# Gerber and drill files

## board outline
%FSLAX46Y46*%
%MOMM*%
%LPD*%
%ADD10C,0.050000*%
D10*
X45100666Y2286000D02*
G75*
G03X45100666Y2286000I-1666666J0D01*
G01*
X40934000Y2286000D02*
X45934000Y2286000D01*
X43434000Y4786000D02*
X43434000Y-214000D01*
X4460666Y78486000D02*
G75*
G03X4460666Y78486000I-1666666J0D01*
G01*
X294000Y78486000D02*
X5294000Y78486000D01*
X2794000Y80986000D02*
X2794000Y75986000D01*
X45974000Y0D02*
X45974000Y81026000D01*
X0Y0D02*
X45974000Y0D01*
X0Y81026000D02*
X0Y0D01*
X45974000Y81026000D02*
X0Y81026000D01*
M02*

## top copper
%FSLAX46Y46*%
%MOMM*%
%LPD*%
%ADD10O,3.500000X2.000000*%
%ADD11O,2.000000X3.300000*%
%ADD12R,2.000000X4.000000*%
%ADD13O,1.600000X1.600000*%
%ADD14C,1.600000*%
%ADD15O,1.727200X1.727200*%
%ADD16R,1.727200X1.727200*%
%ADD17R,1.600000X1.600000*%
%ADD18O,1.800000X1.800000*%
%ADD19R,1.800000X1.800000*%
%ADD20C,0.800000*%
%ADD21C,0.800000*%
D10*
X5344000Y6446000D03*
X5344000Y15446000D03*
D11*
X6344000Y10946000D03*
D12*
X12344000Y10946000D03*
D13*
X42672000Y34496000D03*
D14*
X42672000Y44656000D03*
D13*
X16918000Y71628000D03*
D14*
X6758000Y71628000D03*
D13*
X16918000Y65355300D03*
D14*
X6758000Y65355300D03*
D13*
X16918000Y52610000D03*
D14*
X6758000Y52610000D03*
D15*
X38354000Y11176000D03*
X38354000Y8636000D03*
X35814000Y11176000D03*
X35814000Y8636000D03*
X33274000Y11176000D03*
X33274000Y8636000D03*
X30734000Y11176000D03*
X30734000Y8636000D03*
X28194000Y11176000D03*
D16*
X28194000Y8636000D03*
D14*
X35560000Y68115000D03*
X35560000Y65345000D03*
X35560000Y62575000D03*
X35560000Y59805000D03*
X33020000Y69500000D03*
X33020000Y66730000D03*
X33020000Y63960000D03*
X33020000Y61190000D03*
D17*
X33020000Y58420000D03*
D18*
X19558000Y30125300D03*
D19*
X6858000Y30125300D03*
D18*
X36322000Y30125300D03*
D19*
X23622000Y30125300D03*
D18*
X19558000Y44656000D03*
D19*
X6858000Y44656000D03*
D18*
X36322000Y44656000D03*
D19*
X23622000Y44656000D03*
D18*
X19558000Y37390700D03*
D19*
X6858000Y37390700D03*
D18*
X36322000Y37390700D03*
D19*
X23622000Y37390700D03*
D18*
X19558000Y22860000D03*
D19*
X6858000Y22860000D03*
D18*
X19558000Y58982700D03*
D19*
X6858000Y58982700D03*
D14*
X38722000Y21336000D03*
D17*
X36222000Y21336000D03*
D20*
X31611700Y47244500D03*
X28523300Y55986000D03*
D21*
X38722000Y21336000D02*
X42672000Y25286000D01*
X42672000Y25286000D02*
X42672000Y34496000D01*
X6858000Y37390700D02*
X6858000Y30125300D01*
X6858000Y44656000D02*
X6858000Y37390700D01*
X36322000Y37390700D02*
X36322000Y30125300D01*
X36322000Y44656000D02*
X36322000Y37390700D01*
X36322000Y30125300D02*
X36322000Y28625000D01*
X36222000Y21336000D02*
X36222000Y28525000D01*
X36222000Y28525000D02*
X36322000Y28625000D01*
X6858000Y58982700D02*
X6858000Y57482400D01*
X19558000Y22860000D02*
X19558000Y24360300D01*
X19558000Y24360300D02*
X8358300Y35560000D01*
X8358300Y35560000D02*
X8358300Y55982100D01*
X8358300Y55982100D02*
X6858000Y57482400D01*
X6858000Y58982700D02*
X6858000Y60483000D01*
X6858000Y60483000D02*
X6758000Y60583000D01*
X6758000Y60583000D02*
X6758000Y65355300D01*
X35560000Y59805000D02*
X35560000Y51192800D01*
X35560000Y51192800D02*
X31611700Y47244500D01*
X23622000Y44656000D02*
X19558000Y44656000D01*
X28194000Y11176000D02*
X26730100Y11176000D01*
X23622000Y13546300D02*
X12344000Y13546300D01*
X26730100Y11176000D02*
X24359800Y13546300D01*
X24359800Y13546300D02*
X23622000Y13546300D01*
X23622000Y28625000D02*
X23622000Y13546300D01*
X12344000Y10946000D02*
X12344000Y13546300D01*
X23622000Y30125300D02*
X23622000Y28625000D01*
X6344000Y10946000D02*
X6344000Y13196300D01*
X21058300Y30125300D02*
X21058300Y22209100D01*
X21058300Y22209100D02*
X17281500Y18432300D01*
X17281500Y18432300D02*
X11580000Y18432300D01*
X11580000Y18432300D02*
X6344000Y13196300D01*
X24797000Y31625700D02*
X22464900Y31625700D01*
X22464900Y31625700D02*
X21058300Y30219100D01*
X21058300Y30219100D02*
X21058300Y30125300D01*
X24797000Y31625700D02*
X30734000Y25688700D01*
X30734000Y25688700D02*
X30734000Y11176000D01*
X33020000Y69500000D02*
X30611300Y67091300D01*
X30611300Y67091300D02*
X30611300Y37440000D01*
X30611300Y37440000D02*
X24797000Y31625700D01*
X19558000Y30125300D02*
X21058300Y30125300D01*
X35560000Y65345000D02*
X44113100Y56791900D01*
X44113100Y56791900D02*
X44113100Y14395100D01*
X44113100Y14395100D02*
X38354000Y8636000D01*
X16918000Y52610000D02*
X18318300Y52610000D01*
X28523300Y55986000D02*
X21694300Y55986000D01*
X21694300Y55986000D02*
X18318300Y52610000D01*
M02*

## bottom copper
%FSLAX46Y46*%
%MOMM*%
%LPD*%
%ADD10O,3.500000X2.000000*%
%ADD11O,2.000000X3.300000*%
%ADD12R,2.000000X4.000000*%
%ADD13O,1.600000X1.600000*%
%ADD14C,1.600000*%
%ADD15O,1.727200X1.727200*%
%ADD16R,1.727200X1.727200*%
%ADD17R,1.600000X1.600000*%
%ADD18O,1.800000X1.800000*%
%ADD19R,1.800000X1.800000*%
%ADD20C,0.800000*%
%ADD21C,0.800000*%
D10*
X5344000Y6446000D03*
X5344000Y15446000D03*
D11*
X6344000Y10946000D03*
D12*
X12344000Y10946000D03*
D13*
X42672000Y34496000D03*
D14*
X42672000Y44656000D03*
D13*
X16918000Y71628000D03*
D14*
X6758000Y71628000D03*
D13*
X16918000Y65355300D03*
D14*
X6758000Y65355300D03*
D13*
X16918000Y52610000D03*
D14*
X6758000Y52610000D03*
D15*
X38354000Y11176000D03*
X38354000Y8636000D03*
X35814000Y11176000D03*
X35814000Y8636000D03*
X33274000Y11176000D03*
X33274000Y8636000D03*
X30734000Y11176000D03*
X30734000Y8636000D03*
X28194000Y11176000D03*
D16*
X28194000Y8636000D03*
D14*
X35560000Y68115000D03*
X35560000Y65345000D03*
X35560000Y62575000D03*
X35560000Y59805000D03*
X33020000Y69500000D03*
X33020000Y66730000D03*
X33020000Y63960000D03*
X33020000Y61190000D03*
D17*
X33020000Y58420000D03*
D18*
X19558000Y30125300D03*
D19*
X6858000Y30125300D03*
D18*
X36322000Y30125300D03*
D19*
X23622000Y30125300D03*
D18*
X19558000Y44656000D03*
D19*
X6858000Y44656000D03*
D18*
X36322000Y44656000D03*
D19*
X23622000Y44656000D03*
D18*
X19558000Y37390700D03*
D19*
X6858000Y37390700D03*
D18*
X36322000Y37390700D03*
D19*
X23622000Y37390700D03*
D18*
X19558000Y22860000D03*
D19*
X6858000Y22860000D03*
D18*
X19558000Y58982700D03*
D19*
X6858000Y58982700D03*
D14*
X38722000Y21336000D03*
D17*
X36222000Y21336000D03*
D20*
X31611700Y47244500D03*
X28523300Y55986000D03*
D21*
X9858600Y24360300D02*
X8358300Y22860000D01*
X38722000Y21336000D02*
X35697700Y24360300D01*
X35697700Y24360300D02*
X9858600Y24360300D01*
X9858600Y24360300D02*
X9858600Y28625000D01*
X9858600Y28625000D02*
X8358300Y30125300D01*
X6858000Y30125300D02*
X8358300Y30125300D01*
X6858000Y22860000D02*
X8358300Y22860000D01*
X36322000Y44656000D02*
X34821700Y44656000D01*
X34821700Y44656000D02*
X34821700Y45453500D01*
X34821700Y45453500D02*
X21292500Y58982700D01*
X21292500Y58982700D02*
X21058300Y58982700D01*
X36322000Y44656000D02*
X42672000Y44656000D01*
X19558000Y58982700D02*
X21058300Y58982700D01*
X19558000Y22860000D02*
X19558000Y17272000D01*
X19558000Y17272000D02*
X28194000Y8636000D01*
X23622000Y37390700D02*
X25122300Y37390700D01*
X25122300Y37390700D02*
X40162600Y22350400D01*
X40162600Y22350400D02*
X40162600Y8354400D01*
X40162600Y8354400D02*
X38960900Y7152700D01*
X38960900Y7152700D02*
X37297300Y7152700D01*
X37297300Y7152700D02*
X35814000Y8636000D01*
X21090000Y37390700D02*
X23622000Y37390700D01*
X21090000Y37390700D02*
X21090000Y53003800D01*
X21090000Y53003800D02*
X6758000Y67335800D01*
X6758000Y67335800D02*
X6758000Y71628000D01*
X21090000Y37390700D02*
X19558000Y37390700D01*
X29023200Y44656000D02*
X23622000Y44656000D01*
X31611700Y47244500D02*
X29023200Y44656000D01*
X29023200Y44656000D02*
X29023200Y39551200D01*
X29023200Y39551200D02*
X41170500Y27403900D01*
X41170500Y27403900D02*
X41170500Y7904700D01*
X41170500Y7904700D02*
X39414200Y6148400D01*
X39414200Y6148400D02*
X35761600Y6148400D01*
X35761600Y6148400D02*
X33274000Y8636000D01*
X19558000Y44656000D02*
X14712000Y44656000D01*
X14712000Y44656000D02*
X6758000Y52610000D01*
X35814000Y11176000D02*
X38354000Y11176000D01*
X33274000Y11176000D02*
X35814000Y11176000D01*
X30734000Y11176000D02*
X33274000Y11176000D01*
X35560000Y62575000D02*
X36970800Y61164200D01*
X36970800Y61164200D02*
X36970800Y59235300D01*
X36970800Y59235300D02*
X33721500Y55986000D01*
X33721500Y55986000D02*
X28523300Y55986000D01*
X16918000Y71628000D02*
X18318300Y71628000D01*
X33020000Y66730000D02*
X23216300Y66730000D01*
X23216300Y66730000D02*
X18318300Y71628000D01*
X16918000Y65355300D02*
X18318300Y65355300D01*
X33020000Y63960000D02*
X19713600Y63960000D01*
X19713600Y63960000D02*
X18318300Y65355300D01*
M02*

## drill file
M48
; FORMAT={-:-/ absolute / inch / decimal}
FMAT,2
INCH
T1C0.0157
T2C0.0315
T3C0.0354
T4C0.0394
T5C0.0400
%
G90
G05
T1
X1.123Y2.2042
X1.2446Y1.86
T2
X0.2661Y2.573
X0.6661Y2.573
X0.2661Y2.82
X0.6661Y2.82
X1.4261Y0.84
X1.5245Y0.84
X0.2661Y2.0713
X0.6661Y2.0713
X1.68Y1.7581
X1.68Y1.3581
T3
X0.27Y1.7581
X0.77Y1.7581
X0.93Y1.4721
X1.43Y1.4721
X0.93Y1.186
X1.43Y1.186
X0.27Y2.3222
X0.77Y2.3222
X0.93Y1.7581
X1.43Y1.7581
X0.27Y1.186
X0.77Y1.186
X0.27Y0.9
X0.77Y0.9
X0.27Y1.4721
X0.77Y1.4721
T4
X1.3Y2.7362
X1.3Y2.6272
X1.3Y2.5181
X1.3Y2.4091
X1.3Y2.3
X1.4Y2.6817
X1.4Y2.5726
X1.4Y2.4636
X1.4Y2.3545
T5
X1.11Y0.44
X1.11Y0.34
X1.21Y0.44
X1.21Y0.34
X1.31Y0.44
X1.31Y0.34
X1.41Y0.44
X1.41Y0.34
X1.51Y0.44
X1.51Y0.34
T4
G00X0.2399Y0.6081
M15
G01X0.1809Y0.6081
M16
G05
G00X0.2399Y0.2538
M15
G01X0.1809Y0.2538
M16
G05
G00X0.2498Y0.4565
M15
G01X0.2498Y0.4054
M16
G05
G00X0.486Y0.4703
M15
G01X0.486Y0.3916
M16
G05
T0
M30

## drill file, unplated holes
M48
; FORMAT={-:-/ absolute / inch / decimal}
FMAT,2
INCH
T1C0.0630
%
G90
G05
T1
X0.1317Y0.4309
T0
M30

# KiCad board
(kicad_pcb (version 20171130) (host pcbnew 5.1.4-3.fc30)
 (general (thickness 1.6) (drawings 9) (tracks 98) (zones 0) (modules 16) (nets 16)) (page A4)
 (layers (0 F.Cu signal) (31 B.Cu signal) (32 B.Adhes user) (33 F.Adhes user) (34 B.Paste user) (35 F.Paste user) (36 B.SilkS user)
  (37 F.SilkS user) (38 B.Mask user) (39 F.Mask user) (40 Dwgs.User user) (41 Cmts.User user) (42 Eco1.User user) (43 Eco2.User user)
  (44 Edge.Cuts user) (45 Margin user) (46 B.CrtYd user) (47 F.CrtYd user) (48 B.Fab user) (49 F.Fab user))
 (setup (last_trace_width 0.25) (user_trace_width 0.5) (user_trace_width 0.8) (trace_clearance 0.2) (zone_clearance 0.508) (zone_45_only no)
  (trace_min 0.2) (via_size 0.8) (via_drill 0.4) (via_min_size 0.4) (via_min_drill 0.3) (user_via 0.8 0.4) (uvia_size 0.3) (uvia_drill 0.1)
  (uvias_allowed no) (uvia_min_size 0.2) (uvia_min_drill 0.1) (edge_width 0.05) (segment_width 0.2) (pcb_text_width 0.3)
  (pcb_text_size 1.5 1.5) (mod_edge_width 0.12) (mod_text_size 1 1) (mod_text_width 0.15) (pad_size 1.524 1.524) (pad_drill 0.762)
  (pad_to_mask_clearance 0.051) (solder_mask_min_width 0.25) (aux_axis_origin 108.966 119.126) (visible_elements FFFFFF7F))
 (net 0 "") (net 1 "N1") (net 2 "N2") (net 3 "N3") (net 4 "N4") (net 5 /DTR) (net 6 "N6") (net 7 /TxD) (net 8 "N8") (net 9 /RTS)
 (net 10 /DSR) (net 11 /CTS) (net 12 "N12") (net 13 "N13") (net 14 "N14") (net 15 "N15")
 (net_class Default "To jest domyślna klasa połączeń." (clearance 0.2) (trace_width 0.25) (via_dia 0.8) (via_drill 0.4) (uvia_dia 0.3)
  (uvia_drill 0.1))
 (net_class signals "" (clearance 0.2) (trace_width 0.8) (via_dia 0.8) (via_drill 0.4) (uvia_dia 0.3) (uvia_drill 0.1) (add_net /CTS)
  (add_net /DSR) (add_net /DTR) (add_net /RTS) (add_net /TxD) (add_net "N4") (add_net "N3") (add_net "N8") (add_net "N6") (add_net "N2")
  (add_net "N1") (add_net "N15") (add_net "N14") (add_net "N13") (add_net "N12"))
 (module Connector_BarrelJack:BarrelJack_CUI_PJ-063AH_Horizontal (layer F.Cu) (at 121.31 108.18 270)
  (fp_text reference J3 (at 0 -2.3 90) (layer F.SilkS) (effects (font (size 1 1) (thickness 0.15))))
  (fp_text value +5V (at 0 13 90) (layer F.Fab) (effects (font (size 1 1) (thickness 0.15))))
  (pad "" np_thru_hole circle (at 0 9 270) (size 1.6 1.6) (drill 1.6) (layers *.Cu *.Mask))
  (pad MP thru_hole oval (at 4.5 7 270) (size 2 3.5) (drill oval 1 2.5) (layers *.Cu *.Mask))
  (pad MP thru_hole oval (at -4.5 7 270) (size 2 3.5) (drill oval 1 2.5) (layers *.Cu *.Mask))
  (pad 2 thru_hole oval (at 0 6 270) (size 3.3 2) (drill oval 2.3 1) (layers *.Cu *.Mask) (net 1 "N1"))
  (pad 1 thru_hole rect (at 0 0 270) (size 4 2) (drill oval 3 1) (layers *.Cu *.Mask) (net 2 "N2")))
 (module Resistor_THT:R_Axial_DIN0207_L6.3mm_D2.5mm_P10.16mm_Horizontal (layer F.Cu) (at 151.638 74.47 270)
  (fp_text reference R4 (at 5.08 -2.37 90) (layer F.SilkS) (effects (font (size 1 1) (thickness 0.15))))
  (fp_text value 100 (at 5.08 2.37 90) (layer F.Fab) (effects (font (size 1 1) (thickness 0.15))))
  (pad 2 thru_hole oval (at 10.16 0 270) (size 1.6 1.6) (drill 0.8) (layers *.Cu *.Mask) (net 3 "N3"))
  (pad 1 thru_hole circle (at 0 0 270) (size 1.6 1.6) (drill 0.8) (layers *.Cu *.Mask) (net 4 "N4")))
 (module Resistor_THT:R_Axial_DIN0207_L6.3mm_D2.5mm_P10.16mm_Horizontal (layer F.Cu) (at 115.724 47.498)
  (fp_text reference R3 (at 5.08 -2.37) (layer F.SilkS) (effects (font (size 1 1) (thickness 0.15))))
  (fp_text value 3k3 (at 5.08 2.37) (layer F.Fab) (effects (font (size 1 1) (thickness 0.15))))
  (pad 2 thru_hole oval (at 10.16 0) (size 1.6 1.6) (drill 0.8) (layers *.Cu *.Mask) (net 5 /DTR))
  (pad 1 thru_hole circle (at 0 0) (size 1.6 1.6) (drill 0.8) (layers *.Cu *.Mask) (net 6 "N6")))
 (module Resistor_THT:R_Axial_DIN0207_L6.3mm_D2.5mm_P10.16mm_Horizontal (layer F.Cu) (at 115.724 53.7707)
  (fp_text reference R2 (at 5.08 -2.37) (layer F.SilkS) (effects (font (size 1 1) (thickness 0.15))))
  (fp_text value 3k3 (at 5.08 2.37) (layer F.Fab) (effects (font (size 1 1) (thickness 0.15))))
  (pad 2 thru_hole oval (at 10.16 0) (size 1.6 1.6) (drill 0.8) (layers *.Cu *.Mask) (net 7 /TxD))
  (pad 1 thru_hole circle (at 0 0) (size 1.6 1.6) (drill 0.8) (layers *.Cu *.Mask) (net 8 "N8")))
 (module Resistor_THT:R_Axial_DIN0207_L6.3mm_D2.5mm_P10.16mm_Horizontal (layer F.Cu) (at 115.724 66.516)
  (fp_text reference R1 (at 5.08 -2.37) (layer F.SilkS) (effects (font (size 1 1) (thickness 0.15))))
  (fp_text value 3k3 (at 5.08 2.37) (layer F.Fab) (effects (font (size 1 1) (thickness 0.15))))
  (pad 2 thru_hole oval (at 10.16 0) (size 1.6 1.6) (drill 0.8) (layers *.Cu *.Mask) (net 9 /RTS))
  (pad 1 thru_hole circle (at 0 0) (size 1.6 1.6) (drill 0.8) (layers *.Cu *.Mask) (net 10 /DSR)))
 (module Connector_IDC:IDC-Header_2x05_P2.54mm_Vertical (layer F.Cu) (at 137.16 110.49 90)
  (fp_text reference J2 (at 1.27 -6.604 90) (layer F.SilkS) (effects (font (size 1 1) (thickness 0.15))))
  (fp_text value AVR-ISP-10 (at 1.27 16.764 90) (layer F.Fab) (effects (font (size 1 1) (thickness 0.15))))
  (pad 10 thru_hole oval (at 2.54 10.16 90) (size 1.7272 1.7272) (drill 1.016) (layers *.Cu *.Mask) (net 1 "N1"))
  (pad 9 thru_hole oval (at 0 10.16 90) (size 1.7272 1.7272) (drill 1.016) (layers *.Cu *.Mask) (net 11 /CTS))
  (pad 8 thru_hole oval (at 2.54 7.62 90) (size 1.7272 1.7272) (drill 1.016) (layers *.Cu *.Mask) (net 1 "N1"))
  (pad 7 thru_hole oval (at 0 7.62 90) (size 1.7272 1.7272) (drill 1.016) (layers *.Cu *.Mask) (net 6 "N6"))
  (pad 6 thru_hole oval (at 2.54 5.08 90) (size 1.7272 1.7272) (drill 1.016) (layers *.Cu *.Mask) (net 1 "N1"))
  (pad 5 thru_hole oval (at 0 5.08 90) (size 1.7272 1.7272) (drill 1.016) (layers *.Cu *.Mask) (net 10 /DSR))
  (pad 4 thru_hole oval (at 2.54 2.54 90) (size 1.7272 1.7272) (drill 1.016) (layers *.Cu *.Mask) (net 1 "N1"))
  (pad 3 thru_hole oval (at 0 2.54 90) (size 1.7272 1.7272) (drill 1.016) (layers *.Cu *.Mask) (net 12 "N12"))
  (pad 2 thru_hole oval (at 2.54 0 90) (size 1.7272 1.7272) (drill 1.016) (layers *.Cu *.Mask) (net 2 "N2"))
  (pad 1 thru_hole rect (at 0 0 90) (size 1.7272 1.7272) (drill 1.016) (layers *.Cu *.Mask) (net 8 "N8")))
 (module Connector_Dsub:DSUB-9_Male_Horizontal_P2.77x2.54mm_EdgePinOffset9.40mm (layer F.Cu) (at 141.986 60.706 90)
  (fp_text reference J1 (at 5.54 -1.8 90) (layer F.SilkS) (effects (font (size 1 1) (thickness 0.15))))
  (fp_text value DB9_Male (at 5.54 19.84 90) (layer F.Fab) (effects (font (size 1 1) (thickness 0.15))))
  (pad 9 thru_hole circle (at 9.695 2.54 90) (size 1.6 1.6) (drill 1) (layers *.Cu *.Mask) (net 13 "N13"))
  (pad 8 thru_hole circle (at 6.925 2.54 90) (size 1.6 1.6) (drill 1) (layers *.Cu *.Mask) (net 11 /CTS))
  (pad 7 thru_hole circle (at 4.155 2.54 90) (size 1.6 1.6) (drill 1) (layers *.Cu *.Mask) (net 9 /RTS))
  (pad 6 thru_hole circle (at 1.385 2.54 90) (size 1.6 1.6) (drill 1) (layers *.Cu *.Mask) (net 10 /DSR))
  (pad 5 thru_hole circle (at 11.08 0 90) (size 1.6 1.6) (drill 1) (layers *.Cu *.Mask) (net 1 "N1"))
  (pad 4 thru_hole circle (at 8.31 0 90) (size 1.6 1.6) (drill 1) (layers *.Cu *.Mask) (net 5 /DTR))
  (pad 3 thru_hole circle (at 5.54 0 90) (size 1.6 1.6) (drill 1) (layers *.Cu *.Mask) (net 7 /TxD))
  (pad 2 thru_hole circle (at 2.77 0 90) (size 1.6 1.6) (drill 1) (layers *.Cu *.Mask) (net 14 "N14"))
  (pad 1 thru_hole rect (at 0 0 90) (size 1.6 1.6) (drill 1) (layers *.Cu *.Mask) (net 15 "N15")))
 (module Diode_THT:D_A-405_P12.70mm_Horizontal (layer F.Cu) (at 115.824 89.0007)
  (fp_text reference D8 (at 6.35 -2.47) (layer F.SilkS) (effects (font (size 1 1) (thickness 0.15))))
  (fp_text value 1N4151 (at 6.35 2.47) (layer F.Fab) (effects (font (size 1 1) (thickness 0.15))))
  (pad 2 thru_hole oval (at 12.7 0) (size 1.8 1.8) (drill 0.9) (layers *.Cu *.Mask) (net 1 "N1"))
  (pad 1 thru_hole rect (at 0 0) (size 1.8 1.8) (drill 0.9) (layers *.Cu *.Mask) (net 3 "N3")))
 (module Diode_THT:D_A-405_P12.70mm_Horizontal (layer F.Cu) (at 132.588 89.0007)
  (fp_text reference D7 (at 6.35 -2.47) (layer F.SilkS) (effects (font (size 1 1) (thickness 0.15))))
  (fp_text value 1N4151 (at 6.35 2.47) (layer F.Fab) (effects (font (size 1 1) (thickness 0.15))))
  (pad 2 thru_hole oval (at 12.7 0) (size 1.8 1.8) (drill 0.9) (layers *.Cu *.Mask) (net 4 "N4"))
  (pad 1 thru_hole rect (at 0 0) (size 1.8 1.8) (drill 0.9) (layers *.Cu *.Mask) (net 2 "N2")))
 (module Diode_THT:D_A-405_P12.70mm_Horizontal (layer F.Cu) (at 115.824 74.47)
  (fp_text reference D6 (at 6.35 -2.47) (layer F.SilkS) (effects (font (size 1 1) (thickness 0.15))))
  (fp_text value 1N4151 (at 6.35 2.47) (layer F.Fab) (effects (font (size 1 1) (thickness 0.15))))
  (pad 2 thru_hole oval (at 12.7 0) (size 1.8 1.8) (drill 0.9) (layers *.Cu *.Mask) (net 10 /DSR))
  (pad 1 thru_hole rect (at 0 0) (size 1.8 1.8) (drill 0.9) (layers *.Cu *.Mask) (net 3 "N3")))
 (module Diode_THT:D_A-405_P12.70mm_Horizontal (layer F.Cu) (at 132.588 74.47)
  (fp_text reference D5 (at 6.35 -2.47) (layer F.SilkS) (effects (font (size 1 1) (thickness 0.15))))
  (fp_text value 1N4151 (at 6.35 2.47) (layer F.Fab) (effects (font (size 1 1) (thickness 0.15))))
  (pad 2 thru_hole oval (at 12.7 0) (size 1.8 1.8) (drill 0.9) (layers *.Cu *.Mask) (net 4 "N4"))
  (pad 1 thru_hole rect (at 0 0) (size 1.8 1.8) (drill 0.9) (layers *.Cu *.Mask) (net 10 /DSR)))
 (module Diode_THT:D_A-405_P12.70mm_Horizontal (layer F.Cu) (at 115.824 81.7353)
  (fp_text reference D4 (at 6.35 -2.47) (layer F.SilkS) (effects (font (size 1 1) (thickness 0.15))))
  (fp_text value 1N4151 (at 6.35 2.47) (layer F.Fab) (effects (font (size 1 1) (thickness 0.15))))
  (pad 2 thru_hole oval (at 12.7 0) (size 1.8 1.8) (drill 0.9) (layers *.Cu *.Mask) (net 6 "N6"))
  (pad 1 thru_hole rect (at 0 0) (size 1.8 1.8) (drill 0.9) (layers *.Cu *.Mask) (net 3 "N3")))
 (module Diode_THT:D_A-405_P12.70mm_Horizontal (layer F.Cu) (at 132.588 81.7353)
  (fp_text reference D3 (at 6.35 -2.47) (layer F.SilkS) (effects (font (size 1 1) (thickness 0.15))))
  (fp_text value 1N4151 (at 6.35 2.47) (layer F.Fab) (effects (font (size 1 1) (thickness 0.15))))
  (pad 2 thru_hole oval (at 12.7 0) (size 1.8 1.8) (drill 0.9) (layers *.Cu *.Mask) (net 4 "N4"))
  (pad 1 thru_hole rect (at 0 0) (size 1.8 1.8) (drill 0.9) (layers *.Cu *.Mask) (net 6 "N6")))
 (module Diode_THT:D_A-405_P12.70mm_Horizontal (layer F.Cu) (at 115.824 96.266)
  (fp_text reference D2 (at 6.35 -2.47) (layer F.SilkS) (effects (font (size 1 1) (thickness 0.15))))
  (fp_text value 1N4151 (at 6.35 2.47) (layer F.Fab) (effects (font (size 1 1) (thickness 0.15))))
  (pad 2 thru_hole oval (at 12.7 0) (size 1.8 1.8) (drill 0.9) (layers *.Cu *.Mask) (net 8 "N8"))
  (pad 1 thru_hole rect (at 0 0) (size 1.8 1.8) (drill 0.9) (layers *.Cu *.Mask) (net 3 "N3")))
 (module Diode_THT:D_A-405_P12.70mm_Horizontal (layer F.Cu) (at 115.824 60.1433)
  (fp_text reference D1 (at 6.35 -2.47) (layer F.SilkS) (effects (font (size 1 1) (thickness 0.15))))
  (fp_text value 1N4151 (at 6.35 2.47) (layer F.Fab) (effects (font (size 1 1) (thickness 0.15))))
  (pad 2 thru_hole oval (at 12.7 0) (size 1.8 1.8) (drill 0.9) (layers *.Cu *.Mask) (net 4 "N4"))
  (pad 1 thru_hole rect (at 0 0) (size 1.8 1.8) (drill 0.9) (layers *.Cu *.Mask) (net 8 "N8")))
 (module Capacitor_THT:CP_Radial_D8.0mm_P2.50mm (layer F.Cu) (at 145.188 97.79)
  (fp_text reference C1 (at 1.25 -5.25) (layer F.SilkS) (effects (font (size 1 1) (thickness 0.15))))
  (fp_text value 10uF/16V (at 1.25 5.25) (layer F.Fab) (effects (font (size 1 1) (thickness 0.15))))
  (pad 2 thru_hole circle (at 2.5 0) (size 1.6 1.6) (drill 0.8) (layers *.Cu *.Mask) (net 3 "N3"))
  (pad 1 thru_hole rect (at 0 0) (size 1.6 1.6) (drill 0.8) (layers *.Cu *.Mask) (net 4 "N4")))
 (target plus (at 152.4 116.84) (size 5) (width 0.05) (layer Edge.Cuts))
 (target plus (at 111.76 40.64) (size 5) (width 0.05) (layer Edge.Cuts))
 (gr_line (start 154.94 119.126) (end 154.94 38.1) (layer Edge.Cuts) (width 0.05))
 (gr_line (start 108.966 119.126) (end 154.94 119.126) (layer Edge.Cuts) (width 0.05))
 (gr_line (start 108.966 38.1) (end 108.966 119.126) (layer Edge.Cuts) (width 0.05))
 (gr_line (start 154.94 38.1) (end 108.966 38.1) (layer Edge.Cuts) (width 0.05))
 (segment (start 118.8246 94.7657) (end 117.3243 96.266) (width 0.8) (layer B.Cu) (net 3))
 (segment (start 147.688 97.79) (end 144.6637 94.7657) (width 0.8) (layer B.Cu) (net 3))
 (segment (start 144.6637 94.7657) (end 118.8246 94.7657) (width 0.8) (layer B.Cu) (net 3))
 (segment (start 118.8246 94.7657) (end 118.8246 90.501) (width 0.8) (layer B.Cu) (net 3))
 (segment (start 118.8246 90.501) (end 117.3243 89.0007) (width 0.8) (layer B.Cu) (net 3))
 (segment (start 115.824 89.0007) (end 117.3243 89.0007) (width 0.8) (layer B.Cu) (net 3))
 (segment (start 147.688 97.79) (end 151.638 93.84) (width 0.8) (layer F.Cu) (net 3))
 (segment (start 151.638 93.84) (end 151.638 84.63) (width 0.8) (layer F.Cu) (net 3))
 (segment (start 115.824 96.266) (end 117.3243 96.266) (width 0.8) (layer B.Cu) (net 3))
 (segment (start 115.824 81.7353) (end 115.824 89.0007) (width 0.8) (layer F.Cu) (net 3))
 (segment (start 115.824 74.47) (end 115.824 81.7353) (width 0.8) (layer F.Cu) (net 3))
 (segment (start 145.288 74.47) (end 143.7877 74.47) (width 0.8) (layer B.Cu) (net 4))
 (segment (start 143.7877 74.47) (end 143.7877 73.6725) (width 0.8) (layer B.Cu) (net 4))
 (segment (start 143.7877 73.6725) (end 130.2585 60.1433) (width 0.8) (layer B.Cu) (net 4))
 (segment (start 130.2585 60.1433) (end 130.0243 60.1433) (width 0.8) (layer B.Cu) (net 4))
 (segment (start 145.288 74.47) (end 151.638 74.47) (width 0.8) (layer B.Cu) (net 4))
 (segment (start 128.524 60.1433) (end 130.0243 60.1433) (width 0.8) (layer B.Cu) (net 4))
 (segment (start 145.288 81.7353) (end 145.288 89.0007) (width 0.8) (layer F.Cu) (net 4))
 (segment (start 145.288 74.47) (end 145.288 81.7353) (width 0.8) (layer F.Cu) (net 4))
 (segment (start 145.288 89.0007) (end 145.288 90.501) (width 0.8) (layer F.Cu) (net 4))
 (segment (start 145.188 97.79) (end 145.188 90.601) (width 0.8) (layer F.Cu) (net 4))
 (segment (start 145.188 90.601) (end 145.288 90.501) (width 0.8) (layer F.Cu) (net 4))
 (segment (start 115.824 60.1433) (end 115.824 61.6436) (width 0.8) (layer F.Cu) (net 8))
 (segment (start 128.524 96.266) (end 128.524 94.7657) (width 0.8) (layer F.Cu) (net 8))
 (segment (start 128.524 94.7657) (end 117.3243 83.566) (width 0.8) (layer F.Cu) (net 8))
 (segment (start 117.3243 83.566) (end 117.3243 63.1439) (width 0.8) (layer F.Cu) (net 8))
 (segment (start 117.3243 63.1439) (end 115.824 61.6436) (width 0.8) (layer F.Cu) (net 8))
 (segment (start 128.524 96.266) (end 128.524 101.854) (width 0.8) (layer B.Cu) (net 8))
 (segment (start 128.524 101.854) (end 137.16 110.49) (width 0.8) (layer B.Cu) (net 8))
 (segment (start 115.824 60.1433) (end 115.824 58.643) (width 0.8) (layer F.Cu) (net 8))
 (segment (start 115.824 58.643) (end 115.724 58.543) (width 0.8) (layer F.Cu) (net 8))
 (segment (start 115.724 58.543) (end 115.724 53.7707) (width 0.8) (layer F.Cu) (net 8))
 (segment (start 132.588 81.7353) (end 134.0883 81.7353) (width 0.8) (layer B.Cu) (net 6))
 (segment (start 134.0883 81.7353) (end 149.1286 96.7756) (width 0.8) (layer B.Cu) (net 6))
 (segment (start 149.1286 96.7756) (end 149.1286 110.7716) (width 0.8) (layer B.Cu) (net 6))
 (segment (start 149.1286 110.7716) (end 147.9269 111.9733) (width 0.8) (layer B.Cu) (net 6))
 (segment (start 147.9269 111.9733) (end 146.2633 111.9733) (width 0.8) (layer B.Cu) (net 6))
 (segment (start 146.2633 111.9733) (end 144.78 110.49) (width 0.8) (layer B.Cu) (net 6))
 (segment (start 130.056 81.7353) (end 132.588 81.7353) (width 0.8) (layer B.Cu) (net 6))
 (segment (start 130.056 81.7353) (end 130.056 66.1222) (width 0.8) (layer B.Cu) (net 6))
 (segment (start 130.056 66.1222) (end 115.724 51.7902) (width 0.8) (layer B.Cu) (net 6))
 (segment (start 115.724 51.7902) (end 115.724 47.498) (width 0.8) (layer B.Cu) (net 6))
 (segment (start 130.056 81.7353) (end 128.524 81.7353) (width 0.8) (layer B.Cu) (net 6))
 (segment (start 137.9892 74.47) (end 132.588 74.47) (width 0.8) (layer B.Cu) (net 10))
 (segment (start 140.5777 71.8815) (end 137.9892 74.47) (width 0.8) (layer B.Cu) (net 10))
 (segment (start 137.9892 74.47) (end 137.9892 79.5748) (width 0.8) (layer B.Cu) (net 10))
 (segment (start 137.9892 79.5748) (end 150.1365 91.7221) (width 0.8) (layer B.Cu) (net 10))
 (segment (start 150.1365 91.7221) (end 150.1365 111.2213) (width 0.8) (layer B.Cu) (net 10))
 (segment (start 150.1365 111.2213) (end 148.3802 112.9776) (width 0.8) (layer B.Cu) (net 10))
 (segment (start 148.3802 112.9776) (end 144.7276 112.9776) (width 0.8) (layer B.Cu) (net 10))
 (segment (start 144.7276 112.9776) (end 142.24 110.49) (width 0.8) (layer B.Cu) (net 10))
 (segment (start 144.526 59.321) (end 144.526 67.9332) (width 0.8) (layer F.Cu) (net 10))
 (segment (start 144.526 67.9332) (end 140.5777 71.8815) (width 0.8) (layer F.Cu) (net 10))
 (segment (start 128.524 74.47) (end 123.678 74.47) (width 0.8) (layer B.Cu) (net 10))
 (segment (start 123.678 74.47) (end 115.724 66.516) (width 0.8) (layer B.Cu) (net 10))
 (segment (start 132.588 74.47) (end 128.524 74.47) (width 0.8) (layer F.Cu) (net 10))
 (via (at 140.5777 71.8815) (size 0.8) (layers F.Cu B.Cu) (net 10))
 (segment (start 137.16 107.95) (end 135.6961 107.95) (width 0.8) (layer F.Cu) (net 2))
 (segment (start 132.588 105.5797) (end 121.31 105.5797) (width 0.8) (layer F.Cu) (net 2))
 (segment (start 135.6961 107.95) (end 133.3258 105.5797) (width 0.8) (layer F.Cu) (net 2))
 (segment (start 133.3258 105.5797) (end 132.588 105.5797) (width 0.8) (layer F.Cu) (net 2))
 (segment (start 132.588 90.501) (end 132.588 105.5797) (width 0.8) (layer F.Cu) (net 2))
 (segment (start 121.31 108.18) (end 121.31 105.5797) (width 0.8) (layer F.Cu) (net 2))
 (segment (start 132.588 89.0007) (end 132.588 90.501) (width 0.8) (layer F.Cu) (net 2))
 (segment (start 115.31 108.18) (end 115.31 105.9297) (width 0.8) (layer F.Cu) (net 1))
 (segment (start 130.0243 89.0007) (end 130.0243 96.9169) (width 0.8) (layer F.Cu) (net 1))
 (segment (start 130.0243 96.9169) (end 126.2475 100.6937) (width 0.8) (layer F.Cu) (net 1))
 (segment (start 126.2475 100.6937) (end 120.546 100.6937) (width 0.8) (layer F.Cu) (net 1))
 (segment (start 120.546 100.6937) (end 115.31 105.9297) (width 0.8) (layer F.Cu) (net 1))
 (segment (start 133.763 87.5003) (end 131.4309 87.5003) (width 0.8) (layer F.Cu) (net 1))
 (segment (start 131.4309 87.5003) (end 130.0243 88.9069) (width 0.8) (layer F.Cu) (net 1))
 (segment (start 130.0243 88.9069) (end 130.0243 89.0007) (width 0.8) (layer F.Cu) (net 1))
 (segment (start 133.763 87.5003) (end 139.7 93.4373) (width 0.8) (layer F.Cu) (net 1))
 (segment (start 139.7 93.4373) (end 139.7 107.95) (width 0.8) (layer F.Cu) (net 1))
 (segment (start 141.986 49.626) (end 139.5773 52.0347) (width 0.8) (layer F.Cu) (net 1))
 (segment (start 139.5773 52.0347) (end 139.5773 81.686) (width 0.8) (layer F.Cu) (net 1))
 (segment (start 139.5773 81.686) (end 133.763 87.5003) (width 0.8) (layer F.Cu) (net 1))
 (segment (start 128.524 89.0007) (end 130.0243 89.0007) (width 0.8) (layer F.Cu) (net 1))
 (segment (start 144.78 107.95) (end 147.32 107.95) (width 0.8) (layer B.Cu) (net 1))
 (segment (start 142.24 107.95) (end 144.78 107.95) (width 0.8) (layer B.Cu) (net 1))
 (segment (start 139.7 107.95) (end 142.24 107.95) (width 0.8) (layer B.Cu) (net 1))
 (segment (start 144.526 53.781) (end 153.0791 62.3341) (width 0.8) (layer F.Cu) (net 11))
 (segment (start 153.0791 62.3341) (end 153.0791 104.7309) (width 0.8) (layer F.Cu) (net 11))
 (segment (start 153.0791 104.7309) (end 147.32 110.49) (width 0.8) (layer F.Cu) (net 11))
 (segment (start 125.884 66.516) (end 127.2843 66.516) (width 0.8) (layer F.Cu) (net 9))
 (segment (start 137.4893 63.14) (end 130.6603 63.14) (width 0.8) (layer F.Cu) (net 9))
 (segment (start 130.6603 63.14) (end 127.2843 66.516) (width 0.8) (layer F.Cu) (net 9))
 (segment (start 144.526 56.551) (end 145.9368 57.9618) (width 0.8) (layer B.Cu) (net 9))
 (segment (start 145.9368 57.9618) (end 145.9368 59.8907) (width 0.8) (layer B.Cu) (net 9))
 (segment (start 145.9368 59.8907) (end 142.6875 63.14) (width 0.8) (layer B.Cu) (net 9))
 (segment (start 142.6875 63.14) (end 137.4893 63.14) (width 0.8) (layer B.Cu) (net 9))
 (via (at 137.4893 63.14) (size 0.8) (layers F.Cu B.Cu) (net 9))
 (segment (start 125.884 47.498) (end 127.2843 47.498) (width 0.8) (layer B.Cu) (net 5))
 (segment (start 141.986 52.396) (end 132.1823 52.396) (width 0.8) (layer B.Cu) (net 5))
 (segment (start 132.1823 52.396) (end 127.2843 47.498) (width 0.8) (layer B.Cu) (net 5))
 (segment (start 125.884 53.7707) (end 127.2843 53.7707) (width 0.8) (layer B.Cu) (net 7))
 (segment (start 141.986 55.166) (end 128.6796 55.166) (width 0.8) (layer B.Cu) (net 7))
 (segment (start 128.6796 55.166) (end 127.2843 53.7707) (width 0.8) (layer B.Cu) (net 7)))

